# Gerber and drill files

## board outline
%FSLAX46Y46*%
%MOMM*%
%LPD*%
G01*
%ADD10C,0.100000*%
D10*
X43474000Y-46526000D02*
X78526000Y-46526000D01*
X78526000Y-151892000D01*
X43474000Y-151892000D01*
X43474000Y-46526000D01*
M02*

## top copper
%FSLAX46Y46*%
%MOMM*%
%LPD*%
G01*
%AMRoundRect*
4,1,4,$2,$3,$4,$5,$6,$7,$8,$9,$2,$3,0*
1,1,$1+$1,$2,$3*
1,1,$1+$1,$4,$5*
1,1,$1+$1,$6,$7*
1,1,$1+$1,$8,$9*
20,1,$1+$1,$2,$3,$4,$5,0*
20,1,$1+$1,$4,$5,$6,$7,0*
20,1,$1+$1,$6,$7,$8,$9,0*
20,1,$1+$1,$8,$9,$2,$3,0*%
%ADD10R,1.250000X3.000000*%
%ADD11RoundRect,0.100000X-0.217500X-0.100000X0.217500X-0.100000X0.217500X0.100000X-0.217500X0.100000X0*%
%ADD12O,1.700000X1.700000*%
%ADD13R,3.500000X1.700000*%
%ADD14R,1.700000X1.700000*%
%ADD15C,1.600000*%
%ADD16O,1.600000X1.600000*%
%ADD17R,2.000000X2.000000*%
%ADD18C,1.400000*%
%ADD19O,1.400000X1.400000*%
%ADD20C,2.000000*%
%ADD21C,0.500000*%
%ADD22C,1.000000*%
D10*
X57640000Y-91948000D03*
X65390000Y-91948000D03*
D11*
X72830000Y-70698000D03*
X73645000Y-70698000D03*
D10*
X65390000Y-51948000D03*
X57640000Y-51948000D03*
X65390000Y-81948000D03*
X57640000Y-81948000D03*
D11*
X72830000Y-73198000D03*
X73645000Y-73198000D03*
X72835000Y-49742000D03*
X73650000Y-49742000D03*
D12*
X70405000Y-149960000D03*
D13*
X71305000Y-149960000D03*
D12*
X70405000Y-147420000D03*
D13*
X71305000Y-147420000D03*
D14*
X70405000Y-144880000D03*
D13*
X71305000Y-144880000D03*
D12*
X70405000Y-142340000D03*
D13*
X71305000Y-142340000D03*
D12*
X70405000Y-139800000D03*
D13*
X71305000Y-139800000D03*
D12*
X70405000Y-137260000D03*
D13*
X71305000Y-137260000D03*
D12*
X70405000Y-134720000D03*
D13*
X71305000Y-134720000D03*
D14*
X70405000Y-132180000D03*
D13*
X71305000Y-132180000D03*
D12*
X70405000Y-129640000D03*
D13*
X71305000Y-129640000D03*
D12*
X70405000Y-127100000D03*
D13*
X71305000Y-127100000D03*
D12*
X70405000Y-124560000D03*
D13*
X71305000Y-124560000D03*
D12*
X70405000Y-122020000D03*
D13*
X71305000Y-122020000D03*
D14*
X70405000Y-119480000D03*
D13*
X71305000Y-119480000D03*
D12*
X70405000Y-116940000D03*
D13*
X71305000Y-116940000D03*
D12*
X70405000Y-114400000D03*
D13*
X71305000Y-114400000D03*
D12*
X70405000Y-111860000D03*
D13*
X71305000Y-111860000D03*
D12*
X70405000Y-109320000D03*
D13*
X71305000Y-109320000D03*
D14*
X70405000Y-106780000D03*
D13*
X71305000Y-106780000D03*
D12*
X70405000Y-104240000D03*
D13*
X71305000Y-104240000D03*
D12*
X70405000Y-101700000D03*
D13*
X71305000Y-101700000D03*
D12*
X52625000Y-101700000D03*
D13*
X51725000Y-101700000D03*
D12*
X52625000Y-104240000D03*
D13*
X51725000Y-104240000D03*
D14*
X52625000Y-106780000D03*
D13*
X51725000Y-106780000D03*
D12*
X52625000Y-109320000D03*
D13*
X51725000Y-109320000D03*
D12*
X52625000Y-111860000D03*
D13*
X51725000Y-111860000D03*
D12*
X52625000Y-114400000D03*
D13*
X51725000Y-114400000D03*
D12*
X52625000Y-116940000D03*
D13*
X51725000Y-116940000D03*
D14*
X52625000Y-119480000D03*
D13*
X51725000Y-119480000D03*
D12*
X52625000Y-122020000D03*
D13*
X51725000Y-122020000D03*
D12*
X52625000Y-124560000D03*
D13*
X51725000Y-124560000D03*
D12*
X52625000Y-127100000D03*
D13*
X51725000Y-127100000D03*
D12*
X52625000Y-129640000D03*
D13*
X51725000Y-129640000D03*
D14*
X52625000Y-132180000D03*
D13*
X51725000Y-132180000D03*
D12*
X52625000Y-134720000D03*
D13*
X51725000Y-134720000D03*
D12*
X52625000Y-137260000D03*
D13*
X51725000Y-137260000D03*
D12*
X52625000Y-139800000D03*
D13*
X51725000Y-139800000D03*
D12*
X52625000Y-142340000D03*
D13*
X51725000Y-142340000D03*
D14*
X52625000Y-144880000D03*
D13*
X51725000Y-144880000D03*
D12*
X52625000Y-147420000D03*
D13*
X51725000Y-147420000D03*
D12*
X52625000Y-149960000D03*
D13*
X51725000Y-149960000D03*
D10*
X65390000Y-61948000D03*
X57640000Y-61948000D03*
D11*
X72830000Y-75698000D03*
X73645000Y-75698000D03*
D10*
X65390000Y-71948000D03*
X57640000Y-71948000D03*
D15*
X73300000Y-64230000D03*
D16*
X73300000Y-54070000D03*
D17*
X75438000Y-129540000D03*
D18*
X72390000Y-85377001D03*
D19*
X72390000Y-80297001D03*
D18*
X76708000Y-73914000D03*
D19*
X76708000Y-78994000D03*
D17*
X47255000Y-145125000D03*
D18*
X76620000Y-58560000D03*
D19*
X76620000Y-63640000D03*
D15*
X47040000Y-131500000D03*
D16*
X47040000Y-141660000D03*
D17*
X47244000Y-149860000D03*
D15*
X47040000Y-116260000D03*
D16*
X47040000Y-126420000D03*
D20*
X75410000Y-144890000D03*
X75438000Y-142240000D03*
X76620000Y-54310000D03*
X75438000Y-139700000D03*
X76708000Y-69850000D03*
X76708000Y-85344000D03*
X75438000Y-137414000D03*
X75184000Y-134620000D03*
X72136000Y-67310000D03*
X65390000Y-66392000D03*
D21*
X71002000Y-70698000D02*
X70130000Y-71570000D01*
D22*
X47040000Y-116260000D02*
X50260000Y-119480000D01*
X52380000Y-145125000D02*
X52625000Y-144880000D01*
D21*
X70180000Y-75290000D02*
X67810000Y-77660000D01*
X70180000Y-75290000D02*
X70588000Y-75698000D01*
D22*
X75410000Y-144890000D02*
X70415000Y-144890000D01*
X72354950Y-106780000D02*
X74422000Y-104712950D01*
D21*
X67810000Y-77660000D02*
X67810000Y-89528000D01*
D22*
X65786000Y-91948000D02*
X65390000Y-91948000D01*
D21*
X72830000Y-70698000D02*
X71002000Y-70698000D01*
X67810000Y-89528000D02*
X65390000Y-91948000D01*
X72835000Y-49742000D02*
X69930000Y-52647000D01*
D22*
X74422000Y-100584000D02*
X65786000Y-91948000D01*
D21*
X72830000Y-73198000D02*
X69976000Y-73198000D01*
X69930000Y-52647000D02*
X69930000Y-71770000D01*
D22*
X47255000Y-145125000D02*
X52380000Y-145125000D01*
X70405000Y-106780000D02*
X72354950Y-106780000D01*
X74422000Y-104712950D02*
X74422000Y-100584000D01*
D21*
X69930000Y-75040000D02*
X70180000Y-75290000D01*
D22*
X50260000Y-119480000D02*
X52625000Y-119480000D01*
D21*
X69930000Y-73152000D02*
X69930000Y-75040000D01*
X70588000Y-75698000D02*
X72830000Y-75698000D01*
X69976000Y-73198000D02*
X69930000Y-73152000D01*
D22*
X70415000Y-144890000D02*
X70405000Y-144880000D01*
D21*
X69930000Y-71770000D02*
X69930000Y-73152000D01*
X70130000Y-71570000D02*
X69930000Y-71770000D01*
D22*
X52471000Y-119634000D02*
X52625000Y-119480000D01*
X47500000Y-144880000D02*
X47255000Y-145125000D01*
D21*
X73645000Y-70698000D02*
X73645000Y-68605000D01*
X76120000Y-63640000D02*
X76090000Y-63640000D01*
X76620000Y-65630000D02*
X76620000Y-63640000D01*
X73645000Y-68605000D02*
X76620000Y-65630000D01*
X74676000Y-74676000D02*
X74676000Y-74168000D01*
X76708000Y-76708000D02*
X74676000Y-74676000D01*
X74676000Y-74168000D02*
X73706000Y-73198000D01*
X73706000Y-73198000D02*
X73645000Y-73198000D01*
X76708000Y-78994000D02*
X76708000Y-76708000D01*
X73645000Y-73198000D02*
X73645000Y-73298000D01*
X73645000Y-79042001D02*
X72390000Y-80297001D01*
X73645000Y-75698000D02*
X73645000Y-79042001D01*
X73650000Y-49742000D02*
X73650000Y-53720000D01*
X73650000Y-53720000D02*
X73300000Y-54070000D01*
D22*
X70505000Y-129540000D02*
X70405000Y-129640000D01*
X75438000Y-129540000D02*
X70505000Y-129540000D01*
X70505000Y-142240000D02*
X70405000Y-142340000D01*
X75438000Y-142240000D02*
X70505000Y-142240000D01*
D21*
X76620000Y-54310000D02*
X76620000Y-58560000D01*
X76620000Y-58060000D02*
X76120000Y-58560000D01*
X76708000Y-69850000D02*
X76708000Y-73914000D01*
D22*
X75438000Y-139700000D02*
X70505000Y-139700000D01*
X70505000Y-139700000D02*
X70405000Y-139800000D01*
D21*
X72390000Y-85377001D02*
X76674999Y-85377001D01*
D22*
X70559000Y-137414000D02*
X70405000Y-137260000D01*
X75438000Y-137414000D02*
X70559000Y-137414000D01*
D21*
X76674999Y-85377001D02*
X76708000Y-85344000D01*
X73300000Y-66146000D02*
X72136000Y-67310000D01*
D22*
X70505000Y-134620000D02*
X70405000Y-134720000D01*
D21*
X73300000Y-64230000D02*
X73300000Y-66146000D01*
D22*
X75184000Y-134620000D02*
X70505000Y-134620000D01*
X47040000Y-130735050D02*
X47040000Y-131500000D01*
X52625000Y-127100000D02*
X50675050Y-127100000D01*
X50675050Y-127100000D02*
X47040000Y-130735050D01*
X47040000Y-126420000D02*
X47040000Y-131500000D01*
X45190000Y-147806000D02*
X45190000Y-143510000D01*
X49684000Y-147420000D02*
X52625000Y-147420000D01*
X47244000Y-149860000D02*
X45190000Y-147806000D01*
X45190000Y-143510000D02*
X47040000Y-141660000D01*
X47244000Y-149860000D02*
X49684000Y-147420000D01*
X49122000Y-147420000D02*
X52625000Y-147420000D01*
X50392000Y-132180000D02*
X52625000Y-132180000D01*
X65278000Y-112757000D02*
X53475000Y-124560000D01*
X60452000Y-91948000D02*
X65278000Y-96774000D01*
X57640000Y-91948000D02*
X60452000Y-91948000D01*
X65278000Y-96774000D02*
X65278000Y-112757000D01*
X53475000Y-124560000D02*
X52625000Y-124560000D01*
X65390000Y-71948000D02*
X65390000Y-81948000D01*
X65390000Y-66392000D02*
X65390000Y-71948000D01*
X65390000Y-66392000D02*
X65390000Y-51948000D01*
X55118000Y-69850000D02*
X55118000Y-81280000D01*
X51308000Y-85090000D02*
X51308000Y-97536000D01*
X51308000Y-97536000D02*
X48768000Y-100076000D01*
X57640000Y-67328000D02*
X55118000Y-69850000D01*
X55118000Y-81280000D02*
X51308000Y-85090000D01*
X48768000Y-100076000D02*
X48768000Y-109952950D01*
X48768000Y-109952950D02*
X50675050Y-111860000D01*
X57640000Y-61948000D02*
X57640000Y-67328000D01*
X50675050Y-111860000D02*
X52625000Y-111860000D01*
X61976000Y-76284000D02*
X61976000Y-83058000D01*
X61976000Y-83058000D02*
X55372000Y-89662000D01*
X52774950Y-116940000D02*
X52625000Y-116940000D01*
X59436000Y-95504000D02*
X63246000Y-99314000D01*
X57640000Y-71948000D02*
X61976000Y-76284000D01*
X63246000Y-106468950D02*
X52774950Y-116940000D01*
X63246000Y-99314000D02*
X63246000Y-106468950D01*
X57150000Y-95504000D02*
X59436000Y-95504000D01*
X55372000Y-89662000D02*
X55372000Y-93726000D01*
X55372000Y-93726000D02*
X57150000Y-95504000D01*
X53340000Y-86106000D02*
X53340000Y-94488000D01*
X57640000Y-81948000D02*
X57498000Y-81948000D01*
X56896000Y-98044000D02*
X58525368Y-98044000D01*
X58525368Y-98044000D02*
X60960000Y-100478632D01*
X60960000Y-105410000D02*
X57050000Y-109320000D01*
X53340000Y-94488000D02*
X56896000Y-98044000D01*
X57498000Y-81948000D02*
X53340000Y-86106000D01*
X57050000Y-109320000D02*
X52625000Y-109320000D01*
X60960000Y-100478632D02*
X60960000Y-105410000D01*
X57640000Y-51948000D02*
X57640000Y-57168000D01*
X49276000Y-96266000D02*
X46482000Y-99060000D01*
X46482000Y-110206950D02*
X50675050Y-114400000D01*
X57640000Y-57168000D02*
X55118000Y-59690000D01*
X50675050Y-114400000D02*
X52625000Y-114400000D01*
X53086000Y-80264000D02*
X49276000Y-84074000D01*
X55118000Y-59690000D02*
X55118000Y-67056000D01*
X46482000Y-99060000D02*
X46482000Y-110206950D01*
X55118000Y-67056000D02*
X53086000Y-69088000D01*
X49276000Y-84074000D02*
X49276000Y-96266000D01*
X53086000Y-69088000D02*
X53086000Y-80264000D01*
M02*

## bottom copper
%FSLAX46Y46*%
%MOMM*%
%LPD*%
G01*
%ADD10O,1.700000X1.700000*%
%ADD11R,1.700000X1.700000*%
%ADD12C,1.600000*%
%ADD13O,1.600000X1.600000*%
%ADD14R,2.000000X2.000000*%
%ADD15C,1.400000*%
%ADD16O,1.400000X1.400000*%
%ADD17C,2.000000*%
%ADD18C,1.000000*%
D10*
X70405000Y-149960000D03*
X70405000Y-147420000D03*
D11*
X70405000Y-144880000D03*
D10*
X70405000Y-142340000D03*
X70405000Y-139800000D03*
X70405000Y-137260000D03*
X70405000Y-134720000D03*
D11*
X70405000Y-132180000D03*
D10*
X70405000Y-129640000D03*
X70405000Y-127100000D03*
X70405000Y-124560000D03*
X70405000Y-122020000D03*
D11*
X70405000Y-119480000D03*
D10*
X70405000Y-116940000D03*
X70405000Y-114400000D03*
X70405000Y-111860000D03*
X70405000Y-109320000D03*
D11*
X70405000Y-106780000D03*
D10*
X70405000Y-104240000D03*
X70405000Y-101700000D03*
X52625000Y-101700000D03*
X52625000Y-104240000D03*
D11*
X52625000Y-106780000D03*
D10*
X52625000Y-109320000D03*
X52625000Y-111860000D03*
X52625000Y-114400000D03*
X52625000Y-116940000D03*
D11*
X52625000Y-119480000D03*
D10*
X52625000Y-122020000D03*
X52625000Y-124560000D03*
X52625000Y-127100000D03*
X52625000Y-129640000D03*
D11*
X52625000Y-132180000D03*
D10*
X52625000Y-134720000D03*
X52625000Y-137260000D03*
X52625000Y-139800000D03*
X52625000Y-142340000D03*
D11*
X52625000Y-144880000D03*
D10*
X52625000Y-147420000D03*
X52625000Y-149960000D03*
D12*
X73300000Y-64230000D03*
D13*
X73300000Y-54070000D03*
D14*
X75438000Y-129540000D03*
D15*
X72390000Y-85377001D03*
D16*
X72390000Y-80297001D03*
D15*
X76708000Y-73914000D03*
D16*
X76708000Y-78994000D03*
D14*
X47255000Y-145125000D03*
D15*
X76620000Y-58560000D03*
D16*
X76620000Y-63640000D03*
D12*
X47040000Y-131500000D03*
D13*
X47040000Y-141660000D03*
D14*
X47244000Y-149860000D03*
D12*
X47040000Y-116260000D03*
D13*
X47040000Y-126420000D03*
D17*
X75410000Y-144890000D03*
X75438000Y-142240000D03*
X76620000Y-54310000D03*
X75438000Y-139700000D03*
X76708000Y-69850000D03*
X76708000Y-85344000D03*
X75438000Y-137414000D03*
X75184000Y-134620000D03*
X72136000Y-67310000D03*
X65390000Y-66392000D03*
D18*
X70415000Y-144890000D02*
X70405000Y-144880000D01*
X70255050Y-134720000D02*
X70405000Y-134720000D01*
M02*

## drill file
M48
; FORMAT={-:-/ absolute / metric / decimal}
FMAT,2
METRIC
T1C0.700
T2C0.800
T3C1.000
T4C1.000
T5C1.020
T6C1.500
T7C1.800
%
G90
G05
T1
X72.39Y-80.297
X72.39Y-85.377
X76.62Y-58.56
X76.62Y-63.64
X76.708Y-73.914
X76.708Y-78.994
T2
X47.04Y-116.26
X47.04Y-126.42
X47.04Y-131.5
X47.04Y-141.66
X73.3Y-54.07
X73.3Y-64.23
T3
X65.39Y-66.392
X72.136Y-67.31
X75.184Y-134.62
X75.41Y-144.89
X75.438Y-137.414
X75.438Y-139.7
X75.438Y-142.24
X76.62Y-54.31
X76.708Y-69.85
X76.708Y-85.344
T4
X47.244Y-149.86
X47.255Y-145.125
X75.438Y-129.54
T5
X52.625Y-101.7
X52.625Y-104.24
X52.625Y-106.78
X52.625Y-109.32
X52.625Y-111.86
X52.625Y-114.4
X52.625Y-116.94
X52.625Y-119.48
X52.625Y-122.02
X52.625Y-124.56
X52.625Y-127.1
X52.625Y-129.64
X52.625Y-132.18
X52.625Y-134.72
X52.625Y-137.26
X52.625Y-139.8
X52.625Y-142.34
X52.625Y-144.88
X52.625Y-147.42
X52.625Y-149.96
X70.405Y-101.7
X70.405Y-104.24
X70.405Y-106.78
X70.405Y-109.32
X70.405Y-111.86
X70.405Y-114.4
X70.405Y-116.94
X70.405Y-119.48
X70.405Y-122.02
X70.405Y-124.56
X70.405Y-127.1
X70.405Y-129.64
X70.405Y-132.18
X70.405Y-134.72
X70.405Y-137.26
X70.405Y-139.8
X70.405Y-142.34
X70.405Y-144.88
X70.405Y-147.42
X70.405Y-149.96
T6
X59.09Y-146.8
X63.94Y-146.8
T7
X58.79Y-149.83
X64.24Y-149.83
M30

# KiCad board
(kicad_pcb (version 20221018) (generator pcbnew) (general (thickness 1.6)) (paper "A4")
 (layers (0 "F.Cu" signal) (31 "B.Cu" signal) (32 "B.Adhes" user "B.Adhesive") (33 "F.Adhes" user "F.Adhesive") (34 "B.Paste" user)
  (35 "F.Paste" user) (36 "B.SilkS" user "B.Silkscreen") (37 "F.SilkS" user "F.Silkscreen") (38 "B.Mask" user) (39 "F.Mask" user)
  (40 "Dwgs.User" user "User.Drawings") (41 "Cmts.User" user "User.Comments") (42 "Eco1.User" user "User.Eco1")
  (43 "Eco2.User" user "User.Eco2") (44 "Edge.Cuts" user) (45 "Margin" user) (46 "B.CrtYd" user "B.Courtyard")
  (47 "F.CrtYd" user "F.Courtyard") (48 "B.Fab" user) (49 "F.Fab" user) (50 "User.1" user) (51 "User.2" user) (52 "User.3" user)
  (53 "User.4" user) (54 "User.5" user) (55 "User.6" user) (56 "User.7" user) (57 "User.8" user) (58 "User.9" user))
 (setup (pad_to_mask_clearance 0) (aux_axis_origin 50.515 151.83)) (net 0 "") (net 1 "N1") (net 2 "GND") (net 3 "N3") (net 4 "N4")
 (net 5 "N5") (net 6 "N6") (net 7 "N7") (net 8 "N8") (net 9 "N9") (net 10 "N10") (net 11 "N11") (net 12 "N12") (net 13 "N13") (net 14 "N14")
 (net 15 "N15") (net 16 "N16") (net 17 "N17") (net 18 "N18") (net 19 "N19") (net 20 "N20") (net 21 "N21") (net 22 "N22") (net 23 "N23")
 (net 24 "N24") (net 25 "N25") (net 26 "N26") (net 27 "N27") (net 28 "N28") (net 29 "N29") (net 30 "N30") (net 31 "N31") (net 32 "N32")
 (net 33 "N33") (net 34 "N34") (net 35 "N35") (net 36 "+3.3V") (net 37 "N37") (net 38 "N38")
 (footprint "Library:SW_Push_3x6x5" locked (layer "F.Cu") (at 61.515 91.948)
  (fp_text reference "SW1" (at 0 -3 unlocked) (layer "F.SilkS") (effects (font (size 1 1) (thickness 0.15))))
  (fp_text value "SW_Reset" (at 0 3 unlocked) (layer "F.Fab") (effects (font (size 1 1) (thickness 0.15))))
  (pad "1" smd rect locked (at -3.875 0) (size 1.25 3) (layers "F.Cu" "F.Paste" "F.Mask") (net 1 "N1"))
  (pad "2" smd rect locked (at 3.875 0) (size 1.25 3) (layers "F.Cu" "F.Paste" "F.Mask") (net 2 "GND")))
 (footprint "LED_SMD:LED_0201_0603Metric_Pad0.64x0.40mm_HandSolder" (layer "F.Cu") (at 73.2375 70.698)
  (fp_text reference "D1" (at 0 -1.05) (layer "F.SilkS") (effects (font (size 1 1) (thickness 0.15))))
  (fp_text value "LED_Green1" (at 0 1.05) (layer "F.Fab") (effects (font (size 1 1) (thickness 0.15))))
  (pad "" smd roundrect (at -0.4325 0) (size 0.458 0.36) (layers "F.Paste") (roundrect_rratio 0.25))
  (pad "" smd roundrect (at 0.4325 0) (size 0.458 0.36) (layers "F.Paste") (roundrect_rratio 0.25))
  (pad "1" smd roundrect (at -0.4075 0) (size 0.635 0.4) (layers "F.Cu" "F.Mask") (roundrect_rratio 0.25) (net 2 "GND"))
  (pad "2" smd roundrect (at 0.4075 0) (size 0.635 0.4) (layers "F.Cu" "F.Mask") (roundrect_rratio 0.25) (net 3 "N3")))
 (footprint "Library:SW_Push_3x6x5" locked (layer "F.Cu") (at 61.515 51.948 180)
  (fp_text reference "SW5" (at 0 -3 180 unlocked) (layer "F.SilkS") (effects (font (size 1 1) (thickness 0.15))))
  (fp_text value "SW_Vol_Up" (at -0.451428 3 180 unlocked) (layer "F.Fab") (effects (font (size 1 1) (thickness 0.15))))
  (pad "1" smd rect locked (at -3.875 0 180) (size 1.25 3) (layers "F.Cu" "F.Paste" "F.Mask") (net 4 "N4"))
  (pad "2" smd rect locked (at 3.875 0 180) (size 1.25 3) (layers "F.Cu" "F.Paste" "F.Mask") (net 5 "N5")))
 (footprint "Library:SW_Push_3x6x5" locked (layer "F.Cu") (at 61.515 81.948 180)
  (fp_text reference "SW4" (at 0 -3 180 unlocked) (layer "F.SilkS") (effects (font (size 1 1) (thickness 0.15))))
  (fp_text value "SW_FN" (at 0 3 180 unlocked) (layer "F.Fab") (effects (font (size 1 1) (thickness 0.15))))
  (pad "1" smd rect locked (at -3.875 0 180) (size 1.25 3) (layers "F.Cu" "F.Paste" "F.Mask") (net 4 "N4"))
  (pad "2" smd rect locked (at 3.875 0 180) (size 1.25 3) (layers "F.Cu" "F.Paste" "F.Mask") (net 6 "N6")))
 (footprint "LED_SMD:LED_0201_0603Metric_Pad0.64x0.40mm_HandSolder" (layer "F.Cu") (at 73.2375 73.198)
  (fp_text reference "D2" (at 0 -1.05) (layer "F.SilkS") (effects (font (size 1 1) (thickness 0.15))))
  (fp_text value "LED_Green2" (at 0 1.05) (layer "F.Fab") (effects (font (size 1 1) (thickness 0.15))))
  (pad "" smd roundrect (at -0.4325 0) (size 0.458 0.36) (layers "F.Paste") (roundrect_rratio 0.25))
  (pad "" smd roundrect (at 0.4325 0) (size 0.458 0.36) (layers "F.Paste") (roundrect_rratio 0.25))
  (pad "1" smd roundrect (at -0.4075 0) (size 0.635 0.4) (layers "F.Cu" "F.Mask") (roundrect_rratio 0.25) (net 2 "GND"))
  (pad "2" smd roundrect (at 0.4075 0) (size 0.635 0.4) (layers "F.Cu" "F.Mask") (roundrect_rratio 0.25) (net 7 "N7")))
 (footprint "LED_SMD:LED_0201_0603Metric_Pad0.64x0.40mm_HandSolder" (layer "F.Cu") (at 73.2425 49.742)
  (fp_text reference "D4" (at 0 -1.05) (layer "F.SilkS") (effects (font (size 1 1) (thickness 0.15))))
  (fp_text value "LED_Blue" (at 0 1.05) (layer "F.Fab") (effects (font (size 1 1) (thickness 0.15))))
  (pad "" smd roundrect (at -0.4325 0) (size 0.458 0.36) (layers "F.Paste") (roundrect_rratio 0.25))
  (pad "" smd roundrect (at 0.4325 0) (size 0.458 0.36) (layers "F.Paste") (roundrect_rratio 0.25))
  (pad "1" smd roundrect (at -0.4075 0) (size 0.635 0.4) (layers "F.Cu" "F.Mask") (roundrect_rratio 0.25) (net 2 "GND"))
  (pad "2" smd roundrect (at 0.4075 0) (size 0.635 0.4) (layers "F.Cu" "F.Mask") (roundrect_rratio 0.25) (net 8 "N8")))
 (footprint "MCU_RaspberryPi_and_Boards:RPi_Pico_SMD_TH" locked (layer "F.Cu") (at 61.515 125.83 180)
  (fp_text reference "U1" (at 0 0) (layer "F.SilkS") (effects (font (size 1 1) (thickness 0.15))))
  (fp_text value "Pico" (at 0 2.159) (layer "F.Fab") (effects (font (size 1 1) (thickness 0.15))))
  (pad "" np_thru_hole oval locked (at -2.725 -24 180) (size 1.8 1.8) (drill 1.8) (layers "*.Cu" "*.Mask"))
  (pad "" np_thru_hole oval locked (at -2.425 -20.97 180) (size 1.5 1.5) (drill 1.5) (layers "*.Cu" "*.Mask"))
  (pad "" np_thru_hole oval locked (at 2.425 -20.97 180) (size 1.5 1.5) (drill 1.5) (layers "*.Cu" "*.Mask"))
  (pad "" np_thru_hole oval locked (at 2.725 -24 180) (size 1.8 1.8) (drill 1.8) (layers "*.Cu" "*.Mask"))
  (pad "1" thru_hole oval locked (at -8.89 -24.13 180) (size 1.7 1.7) (drill 1.02) (layers "*.Cu" "*.Mask") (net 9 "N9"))
  (pad "1" smd rect locked (at -8.89 -24.13 180) (size 3.5 1.7) (drill (offset -0.9 0)) (layers "F.Cu" "F.Mask") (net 9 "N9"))
  (pad "2" thru_hole oval locked (at -8.89 -21.59 180) (size 1.7 1.7) (drill 1.02) (layers "*.Cu" "*.Mask") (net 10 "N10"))
  (pad "2" smd rect locked (at -8.89 -21.59 180) (size 3.5 1.7) (drill (offset -0.9 0)) (layers "F.Cu" "F.Mask") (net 10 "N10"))
  (pad "3" thru_hole rect locked (at -8.89 -19.05 180) (size 1.7 1.7) (drill 1.02) (layers "*.Cu" "*.Mask") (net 2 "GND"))
  (pad "3" smd rect locked (at -8.89 -19.05 180) (size 3.5 1.7) (drill (offset -0.9 0)) (layers "F.Cu" "F.Mask") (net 2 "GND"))
  (pad "4" thru_hole oval locked (at -8.89 -16.51 180) (size 1.7 1.7) (drill 1.02) (layers "*.Cu" "*.Mask") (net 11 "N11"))
  (pad "4" smd rect locked (at -8.89 -16.51 180) (size 3.5 1.7) (drill (offset -0.9 0)) (layers "F.Cu" "F.Mask") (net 11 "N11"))
  (pad "5" thru_hole oval locked (at -8.89 -13.97 180) (size 1.7 1.7) (drill 1.02) (layers "*.Cu" "*.Mask") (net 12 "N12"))
  (pad "5" smd rect locked (at -8.89 -13.97 180) (size 3.5 1.7) (drill (offset -0.9 0)) (layers "F.Cu" "F.Mask") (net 12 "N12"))
  (pad "6" thru_hole oval locked (at -8.89 -11.43 180) (size 1.7 1.7) (drill 1.02) (layers "*.Cu" "*.Mask") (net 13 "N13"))
  (pad "6" smd rect locked (at -8.89 -11.43 180) (size 3.5 1.7) (drill (offset -0.9 0)) (layers "F.Cu" "F.Mask") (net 13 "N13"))
  (pad "7" thru_hole oval locked (at -8.89 -8.89 180) (size 1.7 1.7) (drill 1.02) (layers "*.Cu" "*.Mask") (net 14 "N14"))
  (pad "7" smd rect locked (at -8.89 -8.89 180) (size 3.5 1.7) (drill (offset -0.9 0)) (layers "F.Cu" "F.Mask") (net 14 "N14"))
  (pad "8" thru_hole rect locked (at -8.89 -6.35 180) (size 1.7 1.7) (drill 1.02) (layers "*.Cu" "*.Mask") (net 2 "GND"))
  (pad "8" smd rect locked (at -8.89 -6.35 180) (size 3.5 1.7) (drill (offset -0.9 0)) (layers "F.Cu" "F.Mask") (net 2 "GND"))
  (pad "9" thru_hole oval locked (at -8.89 -3.81 180) (size 1.7 1.7) (drill 1.02) (layers "*.Cu" "*.Mask") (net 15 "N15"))
  (pad "9" smd rect locked (at -8.89 -3.81 180) (size 3.5 1.7) (drill (offset -0.9 0)) (layers "F.Cu" "F.Mask") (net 15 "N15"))
  (pad "10" thru_hole oval locked (at -8.89 -1.27 180) (size 1.7 1.7) (drill 1.02) (layers "*.Cu" "*.Mask") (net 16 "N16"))
  (pad "10" smd rect locked (at -8.89 -1.27 180) (size 3.5 1.7) (drill (offset -0.9 0)) (layers "F.Cu" "F.Mask") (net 16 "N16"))
  (pad "11" thru_hole oval locked (at -8.89 1.27 180) (size 1.7 1.7) (drill 1.02) (layers "*.Cu" "*.Mask") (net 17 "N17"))
  (pad "11" smd rect locked (at -8.89 1.27 180) (size 3.5 1.7) (drill (offset -0.9 0)) (layers "F.Cu" "F.Mask") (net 17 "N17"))
  (pad "12" thru_hole oval locked (at -8.89 3.81 180) (size 1.7 1.7) (drill 1.02) (layers "*.Cu" "*.Mask") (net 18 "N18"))
  (pad "12" smd rect locked (at -8.89 3.81 180) (size 3.5 1.7) (drill (offset -0.9 0)) (layers "F.Cu" "F.Mask") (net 18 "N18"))
  (pad "13" thru_hole rect locked (at -8.89 6.35 180) (size 1.7 1.7) (drill 1.02) (layers "*.Cu" "*.Mask") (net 2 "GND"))
  (pad "13" smd rect locked (at -8.89 6.35 180) (size 3.5 1.7) (drill (offset -0.9 0)) (layers "F.Cu" "F.Mask") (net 2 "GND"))
  (pad "14" thru_hole oval locked (at -8.89 8.89 180) (size 1.7 1.7) (drill 1.02) (layers "*.Cu" "*.Mask") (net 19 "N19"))
  (pad "14" smd rect locked (at -8.89 8.89 180) (size 3.5 1.7) (drill (offset -0.9 0)) (layers "F.Cu" "F.Mask") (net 19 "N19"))
  (pad "15" thru_hole oval locked (at -8.89 11.43 180) (size 1.7 1.7) (drill 1.02) (layers "*.Cu" "*.Mask") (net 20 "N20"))
  (pad "15" smd rect locked (at -8.89 11.43 180) (size 3.5 1.7) (drill (offset -0.9 0)) (layers "F.Cu" "F.Mask") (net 20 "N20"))
  (pad "16" thru_hole oval locked (at -8.89 13.97 180) (size 1.7 1.7) (drill 1.02) (layers "*.Cu" "*.Mask") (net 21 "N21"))
  (pad "16" smd rect locked (at -8.89 13.97 180) (size 3.5 1.7) (drill (offset -0.9 0)) (layers "F.Cu" "F.Mask") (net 21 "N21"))
  (pad "17" thru_hole oval locked (at -8.89 16.51 180) (size 1.7 1.7) (drill 1.02) (layers "*.Cu" "*.Mask") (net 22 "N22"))
  (pad "17" smd rect locked (at -8.89 16.51 180) (size 3.5 1.7) (drill (offset -0.9 0)) (layers "F.Cu" "F.Mask") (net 22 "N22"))
  (pad "18" thru_hole rect locked (at -8.89 19.05 180) (size 1.7 1.7) (drill 1.02) (layers "*.Cu" "*.Mask") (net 2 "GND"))
  (pad "18" smd rect locked (at -8.89 19.05 180) (size 3.5 1.7) (drill (offset -0.9 0)) (layers "F.Cu" "F.Mask") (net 2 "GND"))
  (pad "19" thru_hole oval locked (at -8.89 21.59 180) (size 1.7 1.7) (drill 1.02) (layers "*.Cu" "*.Mask") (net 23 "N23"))
  (pad "19" smd rect locked (at -8.89 21.59 180) (size 3.5 1.7) (drill (offset -0.9 0)) (layers "F.Cu" "F.Mask") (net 23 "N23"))
  (pad "20" thru_hole oval locked (at -8.89 24.13 180) (size 1.7 1.7) (drill 1.02) (layers "*.Cu" "*.Mask") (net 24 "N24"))
  (pad "20" smd rect locked (at -8.89 24.13 180) (size 3.5 1.7) (drill (offset -0.9 0)) (layers "F.Cu" "F.Mask") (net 24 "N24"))
  (pad "21" thru_hole oval locked (at 8.89 24.13 180) (size 1.7 1.7) (drill 1.02) (layers "*.Cu" "*.Mask") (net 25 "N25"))
  (pad "21" smd rect locked (at 8.89 24.13 180) (size 3.5 1.7) (drill (offset 0.9 0)) (layers "F.Cu" "F.Mask") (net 25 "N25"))
  (pad "22" thru_hole oval locked (at 8.89 21.59 180) (size 1.7 1.7) (drill 1.02) (layers "*.Cu" "*.Mask") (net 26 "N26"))
  (pad "22" smd rect locked (at 8.89 21.59 180) (size 3.5 1.7) (drill (offset 0.9 0)) (layers "F.Cu" "F.Mask") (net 26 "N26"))
  (pad "23" thru_hole rect locked (at 8.89 19.05 180) (size 1.7 1.7) (drill 1.02) (layers "*.Cu" "*.Mask") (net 2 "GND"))
  (pad "23" smd rect locked (at 8.89 19.05 180) (size 3.5 1.7) (drill (offset 0.9 0)) (layers "F.Cu" "F.Mask") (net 2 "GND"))
  (pad "24" thru_hole oval locked (at 8.89 16.51 180) (size 1.7 1.7) (drill 1.02) (layers "*.Cu" "*.Mask") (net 6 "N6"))
  (pad "24" smd rect locked (at 8.89 16.51 180) (size 3.5 1.7) (drill (offset 0.9 0)) (layers "F.Cu" "F.Mask") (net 6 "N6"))
  (pad "25" thru_hole oval locked (at 8.89 13.97 180) (size 1.7 1.7) (drill 1.02) (layers "*.Cu" "*.Mask") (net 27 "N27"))
  (pad "25" smd rect locked (at 8.89 13.97 180) (size 3.5 1.7) (drill (offset 0.9 0)) (layers "F.Cu" "F.Mask") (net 27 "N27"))
  (pad "26" thru_hole oval locked (at 8.89 11.43 180) (size 1.7 1.7) (drill 1.02) (layers "*.Cu" "*.Mask") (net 5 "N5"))
  (pad "26" smd rect locked (at 8.89 11.43 180) (size 3.5 1.7) (drill (offset 0.9 0)) (layers "F.Cu" "F.Mask") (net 5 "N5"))
  (pad "27" thru_hole oval locked (at 8.89 8.89 180) (size 1.7 1.7) (drill 1.02) (layers "*.Cu" "*.Mask") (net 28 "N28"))
  (pad "27" smd rect locked (at 8.89 8.89 180) (size 3.5 1.7) (drill (offset 0.9 0)) (layers "F.Cu" "F.Mask") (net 28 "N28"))
  (pad "28" thru_hole rect locked (at 8.89 6.35 180) (size 1.7 1.7) (drill 1.02) (layers "*.Cu" "*.Mask") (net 2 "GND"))
  (pad "28" smd rect locked (at 8.89 6.35 180) (size 3.5 1.7) (drill (offset 0.9 0)) (layers "F.Cu" "F.Mask") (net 2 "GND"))
  (pad "29" thru_hole oval locked (at 8.89 3.81 180) (size 1.7 1.7) (drill 1.02) (layers "*.Cu" "*.Mask") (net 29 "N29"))
  (pad "29" smd rect locked (at 8.89 3.81 180) (size 3.5 1.7) (drill (offset 0.9 0)) (layers "F.Cu" "F.Mask") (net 29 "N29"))
  (pad "30" thru_hole oval locked (at 8.89 1.27 180) (size 1.7 1.7) (drill 1.02) (layers "*.Cu" "*.Mask") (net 1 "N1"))
  (pad "30" smd rect locked (at 8.89 1.27 180) (size 3.5 1.7) (drill (offset 0.9 0)) (layers "F.Cu" "F.Mask") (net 1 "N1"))
  (pad "31" thru_hole oval locked (at 8.89 -1.27 180) (size 1.7 1.7) (drill 1.02) (layers "*.Cu" "*.Mask") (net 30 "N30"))
  (pad "31" smd rect locked (at 8.89 -1.27 180) (size 3.5 1.7) (drill (offset 0.9 0)) (layers "F.Cu" "F.Mask") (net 30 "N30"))
  (pad "32" thru_hole oval locked (at 8.89 -3.81 180) (size 1.7 1.7) (drill 1.02) (layers "*.Cu" "*.Mask") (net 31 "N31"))
  (pad "32" smd rect locked (at 8.89 -3.81 180) (size 3.5 1.7) (drill (offset 0.9 0)) (layers "F.Cu" "F.Mask") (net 31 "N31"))
  (pad "33" thru_hole rect locked (at 8.89 -6.35 180) (size 1.7 1.7) (drill 1.02) (layers "*.Cu" "*.Mask") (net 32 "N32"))
  (pad "33" smd rect locked (at 8.89 -6.35 180) (size 3.5 1.7) (drill (offset 0.9 0)) (layers "F.Cu" "F.Mask") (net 32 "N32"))
  (pad "34" thru_hole oval locked (at 8.89 -8.89 180) (size 1.7 1.7) (drill 1.02) (layers "*.Cu" "*.Mask") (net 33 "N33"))
  (pad "34" smd rect locked (at 8.89 -8.89 180) (size 3.5 1.7) (drill (offset 0.9 0)) (layers "F.Cu" "F.Mask") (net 33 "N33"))
  (pad "35" thru_hole oval locked (at 8.89 -11.43 180) (size 1.7 1.7) (drill 1.02) (layers "*.Cu" "*.Mask") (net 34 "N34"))
  (pad "35" smd rect locked (at 8.89 -11.43 180) (size 3.5 1.7) (drill (offset 0.9 0)) (layers "F.Cu" "F.Mask") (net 34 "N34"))
  (pad "36" thru_hole oval locked (at 8.89 -13.97 180) (size 1.7 1.7) (drill 1.02) (layers "*.Cu" "*.Mask") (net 4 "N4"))
  (pad "36" smd rect locked (at 8.89 -13.97 180) (size 3.5 1.7) (drill (offset 0.9 0)) (layers "F.Cu" "F.Mask") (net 4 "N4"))
  (pad "37" thru_hole oval locked (at 8.89 -16.51 180) (size 1.7 1.7) (drill 1.02) (layers "*.Cu" "*.Mask") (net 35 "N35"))
  (pad "37" smd rect locked (at 8.89 -16.51 180) (size 3.5 1.7) (drill (offset 0.9 0)) (layers "F.Cu" "F.Mask") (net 35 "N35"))
  (pad "38" thru_hole rect locked (at 8.89 -19.05 180) (size 1.7 1.7) (drill 1.02) (layers "*.Cu" "*.Mask") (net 2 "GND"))
  (pad "38" smd rect locked (at 8.89 -19.05 180) (size 3.5 1.7) (drill (offset 0.9 0)) (layers "F.Cu" "F.Mask") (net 2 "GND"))
  (pad "39" thru_hole oval locked (at 8.89 -21.59 180) (size 1.7 1.7) (drill 1.02) (layers "*.Cu" "*.Mask") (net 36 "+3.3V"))
  (pad "39" smd rect locked (at 8.89 -21.59 180) (size 3.5 1.7) (drill (offset 0.9 0)) (layers "F.Cu" "F.Mask") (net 36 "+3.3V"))
  (pad "40" thru_hole oval locked (at 8.89 -24.13 180) (size 1.7 1.7) (drill 1.02) (layers "*.Cu" "*.Mask") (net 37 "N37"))
  (pad "40" smd rect locked (at 8.89 -24.13 180) (size 3.5 1.7) (drill (offset 0.9 0)) (layers "F.Cu" "F.Mask") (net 37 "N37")))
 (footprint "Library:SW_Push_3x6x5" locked (layer "F.Cu") (at 61.515 61.948 180)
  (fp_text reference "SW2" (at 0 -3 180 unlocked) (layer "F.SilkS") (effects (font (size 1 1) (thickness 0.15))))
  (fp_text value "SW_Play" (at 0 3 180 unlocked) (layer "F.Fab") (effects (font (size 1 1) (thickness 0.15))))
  (pad "1" smd rect locked (at -3.875 0 180) (size 1.25 3) (layers "F.Cu" "F.Paste" "F.Mask") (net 4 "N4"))
  (pad "2" smd rect locked (at 3.875 0 180) (size 1.25 3) (layers "F.Cu" "F.Paste" "F.Mask") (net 27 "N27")))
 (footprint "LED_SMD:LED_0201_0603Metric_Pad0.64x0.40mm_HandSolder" (layer "F.Cu") (at 73.2375 75.698)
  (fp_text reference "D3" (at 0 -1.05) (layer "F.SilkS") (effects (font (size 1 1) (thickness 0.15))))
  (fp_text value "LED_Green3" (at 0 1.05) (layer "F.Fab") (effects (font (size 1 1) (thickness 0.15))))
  (pad "" smd roundrect (at -0.4325 0) (size 0.458 0.36) (layers "F.Paste") (roundrect_rratio 0.25))
  (pad "" smd roundrect (at 0.4325 0) (size 0.458 0.36) (layers "F.Paste") (roundrect_rratio 0.25))
  (pad "1" smd roundrect (at -0.4075 0) (size 0.635 0.4) (layers "F.Cu" "F.Mask") (roundrect_rratio 0.25) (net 2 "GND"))
  (pad "2" smd roundrect (at 0.4075 0) (size 0.635 0.4) (layers "F.Cu" "F.Mask") (roundrect_rratio 0.25) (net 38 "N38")))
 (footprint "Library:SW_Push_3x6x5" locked (layer "F.Cu") (at 61.515 71.948 180)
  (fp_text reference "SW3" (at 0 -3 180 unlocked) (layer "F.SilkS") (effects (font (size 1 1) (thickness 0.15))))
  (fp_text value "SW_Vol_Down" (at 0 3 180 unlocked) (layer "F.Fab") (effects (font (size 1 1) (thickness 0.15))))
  (pad "1" smd rect locked (at -3.875 0 180) (size 1.25 3) (layers "F.Cu" "F.Paste" "F.Mask") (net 4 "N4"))
  (pad "2" smd rect locked (at 3.875 0 180) (size 1.25 3) (layers "F.Cu" "F.Paste" "F.Mask") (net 28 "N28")))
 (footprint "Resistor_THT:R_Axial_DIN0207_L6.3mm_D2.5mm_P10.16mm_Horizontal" (layer "B.Cu") (at 73.3 64.23 90)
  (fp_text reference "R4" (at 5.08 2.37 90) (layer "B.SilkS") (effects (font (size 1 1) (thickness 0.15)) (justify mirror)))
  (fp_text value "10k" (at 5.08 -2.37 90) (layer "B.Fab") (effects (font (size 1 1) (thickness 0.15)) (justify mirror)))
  (pad "1" thru_hole circle (at 0 0 90) (size 1.6 1.6) (drill 0.8) (layers "*.Cu" "*.Mask") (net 14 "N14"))
  (pad "2" thru_hole oval (at 10.16 0 90) (size 1.6 1.6) (drill 0.8) (layers "*.Cu" "*.Mask") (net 8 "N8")))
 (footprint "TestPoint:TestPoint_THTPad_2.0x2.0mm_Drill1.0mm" (layer "B.Cu") (at 75.438 129.54 180)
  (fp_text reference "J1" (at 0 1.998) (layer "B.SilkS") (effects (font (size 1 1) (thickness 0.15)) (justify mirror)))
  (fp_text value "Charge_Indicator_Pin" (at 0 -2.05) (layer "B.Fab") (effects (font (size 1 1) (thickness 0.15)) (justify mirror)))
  (pad "1" thru_hole rect (at 0 0 180) (size 2 2) (drill 1) (layers "*.Cu" "*.Mask") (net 15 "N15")))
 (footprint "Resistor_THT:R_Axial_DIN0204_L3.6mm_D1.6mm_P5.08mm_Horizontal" (layer "B.Cu") (at 72.39 85.377001 90)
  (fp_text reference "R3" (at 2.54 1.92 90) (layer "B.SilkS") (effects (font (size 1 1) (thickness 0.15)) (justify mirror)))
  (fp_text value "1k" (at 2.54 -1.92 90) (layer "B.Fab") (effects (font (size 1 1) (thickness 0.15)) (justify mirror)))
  (pad "1" thru_hole circle (at 0 0 90) (size 1.4 1.4) (drill 0.7) (layers "*.Cu" "*.Mask") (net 13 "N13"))
  (pad "2" thru_hole oval (at 5.08 0 90) (size 1.4 1.4) (drill 0.7) (layers "*.Cu" "*.Mask") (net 38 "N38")))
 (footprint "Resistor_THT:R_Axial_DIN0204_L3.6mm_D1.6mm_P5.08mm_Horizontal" (layer "B.Cu") (at 76.708 73.914 -90)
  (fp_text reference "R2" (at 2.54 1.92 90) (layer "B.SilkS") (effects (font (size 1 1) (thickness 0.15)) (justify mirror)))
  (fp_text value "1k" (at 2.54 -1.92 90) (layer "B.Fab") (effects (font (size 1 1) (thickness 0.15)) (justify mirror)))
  (pad "1" thru_hole circle (at 0 0 270) (size 1.4 1.4) (drill 0.7) (layers "*.Cu" "*.Mask") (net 12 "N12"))
  (pad "2" thru_hole oval (at 5.08 0 270) (size 1.4 1.4) (drill 0.7) (layers "*.Cu" "*.Mask") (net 7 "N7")))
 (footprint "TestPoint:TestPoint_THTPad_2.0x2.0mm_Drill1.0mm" (layer "B.Cu") (at 47.255 145.125 180)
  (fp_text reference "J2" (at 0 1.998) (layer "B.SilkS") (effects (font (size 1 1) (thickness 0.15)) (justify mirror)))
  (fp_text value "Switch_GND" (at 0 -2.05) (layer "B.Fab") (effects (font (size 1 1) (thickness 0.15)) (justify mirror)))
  (pad "1" thru_hole rect (at 0 0 180) (size 2 2) (drill 1) (layers "*.Cu" "*.Mask") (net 2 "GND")))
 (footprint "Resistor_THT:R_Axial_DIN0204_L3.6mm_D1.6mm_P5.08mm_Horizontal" (layer "B.Cu") (at 76.62 58.56 -90)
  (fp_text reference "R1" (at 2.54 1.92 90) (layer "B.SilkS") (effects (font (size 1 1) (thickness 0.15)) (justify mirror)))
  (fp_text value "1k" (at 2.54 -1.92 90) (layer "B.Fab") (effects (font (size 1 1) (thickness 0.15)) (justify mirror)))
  (pad "1" thru_hole circle (at 0 0 270) (size 1.4 1.4) (drill 0.7) (layers "*.Cu" "*.Mask") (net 11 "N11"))
  (pad "2" thru_hole oval (at 5.08 0 270) (size 1.4 1.4) (drill 0.7) (layers "*.Cu" "*.Mask") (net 3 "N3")))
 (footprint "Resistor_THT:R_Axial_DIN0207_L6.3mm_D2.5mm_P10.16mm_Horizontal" (layer "B.Cu") (at 47.04 131.5 -90)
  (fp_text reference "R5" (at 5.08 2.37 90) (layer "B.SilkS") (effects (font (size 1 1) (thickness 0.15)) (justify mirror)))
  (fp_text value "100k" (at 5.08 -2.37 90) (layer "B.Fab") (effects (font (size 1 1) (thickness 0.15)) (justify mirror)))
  (pad "1" thru_hole circle (at 0 0 270) (size 1.6 1.6) (drill 0.8) (layers "*.Cu" "*.Mask") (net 30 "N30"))
  (pad "2" thru_hole oval (at 10.16 0 270) (size 1.6 1.6) (drill 0.8) (layers "*.Cu" "*.Mask") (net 36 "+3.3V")))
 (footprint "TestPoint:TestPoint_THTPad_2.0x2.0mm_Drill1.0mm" (layer "B.Cu") (at 47.244 149.86 180)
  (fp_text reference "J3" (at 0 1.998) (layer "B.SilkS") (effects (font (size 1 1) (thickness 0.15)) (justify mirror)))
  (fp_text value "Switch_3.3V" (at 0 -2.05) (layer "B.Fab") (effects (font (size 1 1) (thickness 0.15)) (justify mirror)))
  (pad "1" thru_hole rect (at 0 0 180) (size 2 2) (drill 1) (layers "*.Cu" "*.Mask") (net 36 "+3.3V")))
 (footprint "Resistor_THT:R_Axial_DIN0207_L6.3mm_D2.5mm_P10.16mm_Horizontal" (layer "B.Cu") (at 47.04 116.26 -90)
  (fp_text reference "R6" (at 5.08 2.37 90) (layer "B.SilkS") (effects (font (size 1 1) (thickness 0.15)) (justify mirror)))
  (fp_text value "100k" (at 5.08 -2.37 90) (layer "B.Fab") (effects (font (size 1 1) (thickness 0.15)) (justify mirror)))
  (pad "1" thru_hole circle (at 0 0 270) (size 1.6 1.6) (drill 0.8) (layers "*.Cu" "*.Mask") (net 2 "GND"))
  (pad "2" thru_hole oval (at 10.16 0 270) (size 1.6 1.6) (drill 0.8) (layers "*.Cu" "*.Mask") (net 30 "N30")))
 (gr_rect (start 43.474 46.526) (end 78.526 151.892) (stroke (width 0.1) (type default)) (fill none) (layer "Edge.Cuts"))
 (segment (start 71.002 70.698) (end 70.13 71.57) (width 0.5) (layer "F.Cu") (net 2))
 (segment (start 47.04 116.26) (end 50.26 119.48) (width 1) (layer "F.Cu") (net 2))
 (segment (start 52.38 145.125) (end 52.625 144.88) (width 1) (layer "F.Cu") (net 2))
 (segment (start 70.18 75.29) (end 67.81 77.66) (width 0.5) (layer "F.Cu") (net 2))
 (segment (start 70.18 75.29) (end 70.588 75.698) (width 0.5) (layer "F.Cu") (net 2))
 (segment (start 75.41 144.89) (end 70.415 144.89) (width 1) (layer "F.Cu") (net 2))
 (segment (start 72.35495 106.78) (end 74.422 104.71295) (width 1) (layer "F.Cu") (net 2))
 (segment (start 67.81 77.66) (end 67.81 89.528) (width 0.5) (layer "F.Cu") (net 2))
 (segment (start 65.786 91.948) (end 65.39 91.948) (width 1) (layer "F.Cu") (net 2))
 (segment (start 72.83 70.698) (end 71.002 70.698) (width 0.5) (layer "F.Cu") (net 2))
 (segment (start 67.81 89.528) (end 65.39 91.948) (width 0.5) (layer "F.Cu") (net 2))
 (segment (start 72.835 49.742) (end 69.93 52.647) (width 0.5) (layer "F.Cu") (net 2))
 (segment (start 74.422 100.584) (end 65.786 91.948) (width 1) (layer "F.Cu") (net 2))
 (segment (start 72.83 73.198) (end 69.976 73.198) (width 0.5) (layer "F.Cu") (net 2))
 (segment (start 69.93 52.647) (end 69.93 71.77) (width 0.5) (layer "F.Cu") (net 2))
 (segment (start 47.255 145.125) (end 52.38 145.125) (width 1) (layer "F.Cu") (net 2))
 (segment (start 70.405 106.78) (end 72.35495 106.78) (width 1) (layer "F.Cu") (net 2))
 (segment (start 74.422 104.71295) (end 74.422 100.584) (width 1) (layer "F.Cu") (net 2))
 (segment (start 69.93 75.04) (end 70.18 75.29) (width 0.5) (layer "F.Cu") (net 2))
 (segment (start 50.26 119.48) (end 52.625 119.48) (width 1) (layer "F.Cu") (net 2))
 (segment (start 69.93 73.152) (end 69.93 75.04) (width 0.5) (layer "F.Cu") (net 2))
 (segment (start 70.588 75.698) (end 72.83 75.698) (width 0.5) (layer "F.Cu") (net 2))
 (segment (start 69.976 73.198) (end 69.93 73.152) (width 0.5) (layer "F.Cu") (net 2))
 (segment (start 70.415 144.89) (end 70.405 144.88) (width 1) (layer "F.Cu") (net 2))
 (segment (start 69.93 71.77) (end 69.93 73.152) (width 0.5) (layer "F.Cu") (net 2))
 (segment (start 70.13 71.57) (end 69.93 71.77) (width 0.5) (layer "F.Cu") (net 2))
 (segment (start 52.471 119.634) (end 52.625 119.48) (width 1) (layer "F.Cu") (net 2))
 (segment (start 47.5 144.88) (end 47.255 145.125) (width 1) (layer "F.Cu") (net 2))
 (via (at 75.41 144.89) (size 2) (drill 1) (layers "F.Cu" "B.Cu") (free) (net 2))
 (segment (start 70.415 144.89) (end 70.405 144.88) (width 1) (layer "B.Cu") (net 2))
 (segment (start 73.645 70.698) (end 73.645 68.605) (width 0.5) (layer "F.Cu") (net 3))
 (segment (start 76.12 63.64) (end 76.09 63.64) (width 0.5) (layer "F.Cu") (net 3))
 (segment (start 76.62 65.63) (end 76.62 63.64) (width 0.5) (layer "F.Cu") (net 3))
 (segment (start 73.645 68.605) (end 76.62 65.63) (width 0.5) (layer "F.Cu") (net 3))
 (segment (start 74.676 74.676) (end 74.676 74.168) (width 0.5) (layer "F.Cu") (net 7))
 (segment (start 76.708 76.708) (end 74.676 74.676) (width 0.5) (layer "F.Cu") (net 7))
 (segment (start 74.676 74.168) (end 73.706 73.198) (width 0.5) (layer "F.Cu") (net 7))
 (segment (start 73.706 73.198) (end 73.645 73.198) (width 0.5) (layer "F.Cu") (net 7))
 (segment (start 76.708 78.994) (end 76.708 76.708) (width 0.5) (layer "F.Cu") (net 7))
 (segment (start 73.645 73.198) (end 73.645 73.298) (width 0.5) (layer "F.Cu") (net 7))
 (segment (start 73.645 79.042001) (end 72.39 80.297001) (width 0.5) (layer "F.Cu") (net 38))
 (segment (start 73.645 75.698) (end 73.645 79.042001) (width 0.5) (layer "F.Cu") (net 38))
 (segment (start 73.65 49.742) (end 73.65 53.72) (width 0.5) (layer "F.Cu") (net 8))
 (segment (start 73.65 53.72) (end 73.3 54.07) (width 0.5) (layer "F.Cu") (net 8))
 (segment (start 70.505 129.54) (end 70.405 129.64) (width 1) (layer "F.Cu") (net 15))
 (segment (start 75.438 129.54) (end 70.505 129.54) (width 1) (layer "F.Cu") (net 15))
 (segment (start 70.505 142.24) (end 70.405 142.34) (width 1) (layer "F.Cu") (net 11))
 (segment (start 75.438 142.24) (end 70.505 142.24) (width 1) (layer "F.Cu") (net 11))
 (segment (start 76.62 54.31) (end 76.62 58.56) (width 0.5) (layer "F.Cu") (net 11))
 (segment (start 76.62 58.06) (end 76.12 58.56) (width 0.5) (layer "F.Cu") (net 11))
 (via (at 75.438 142.24) (size 2) (drill 1) (layers "F.Cu" "B.Cu") (free) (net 11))
 (via (at 76.62 54.31) (size 2) (drill 1) (layers "F.Cu" "B.Cu") (free) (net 11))
 (segment (start 76.708 69.85) (end 76.708 73.914) (width 0.5) (layer "F.Cu") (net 12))
 (segment (start 75.438 139.7) (end 70.505 139.7) (width 1) (layer "F.Cu") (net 12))
 (segment (start 70.505 139.7) (end 70.405 139.8) (width 1) (layer "F.Cu") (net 12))
 (via (at 75.438 139.7) (size 2) (drill 1) (layers "F.Cu" "B.Cu") (free) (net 12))
 (via (at 76.708 69.85) (size 2) (drill 1) (layers "F.Cu" "B.Cu") (free) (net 12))
 (segment (start 72.39 85.377001) (end 76.674999 85.377001) (width 0.5) (layer "F.Cu") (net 13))
 (segment (start 70.559 137.414) (end 70.405 137.26) (width 1) (layer "F.Cu") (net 13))
 (segment (start 75.438 137.414) (end 70.559 137.414) (width 1) (layer "F.Cu") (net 13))
 (segment (start 76.674999 85.377001) (end 76.708 85.344) (width 0.5) (layer "F.Cu") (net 13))
 (via (at 76.708 85.344) (size 2) (drill 1) (layers "F.Cu" "B.Cu") (free) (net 13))
 (via (at 75.438 137.414) (size 2) (drill 1) (layers "F.Cu" "B.Cu") (free) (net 13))
 (segment (start 73.3 66.146) (end 72.136 67.31) (width 0.5) (layer "F.Cu") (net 14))
 (segment (start 70.505 134.62) (end 70.405 134.72) (width 1) (layer "F.Cu") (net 14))
 (segment (start 73.3 64.23) (end 73.3 66.146) (width 0.5) (layer "F.Cu") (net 14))
 (segment (start 75.184 134.62) (end 70.505 134.62) (width 1) (layer "F.Cu") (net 14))
 (via (at 75.184 134.62) (size 2) (drill 1) (layers "F.Cu" "B.Cu") (free) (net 14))
 (via (at 72.136 67.31) (size 2) (drill 1) (layers "F.Cu" "B.Cu") (free) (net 14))
 (segment (start 70.25505 134.72) (end 70.405 134.72) (width 1) (layer "B.Cu") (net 14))
 (segment (start 47.04 130.73505) (end 47.04 131.5) (width 1) (layer "F.Cu") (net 30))
 (segment (start 52.625 127.1) (end 50.67505 127.1) (width 1) (layer "F.Cu") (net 30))
 (segment (start 50.67505 127.1) (end 47.04 130.73505) (width 1) (layer "F.Cu") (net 30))
 (segment (start 47.04 126.42) (end 47.04 131.5) (width 1) (layer "F.Cu") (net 30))
 (segment (start 45.19 147.806) (end 45.19 143.51) (width 1) (layer "F.Cu") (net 36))
 (segment (start 49.684 147.42) (end 52.625 147.42) (width 1) (layer "F.Cu") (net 36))
 (segment (start 47.244 149.86) (end 45.19 147.806) (width 1) (layer "F.Cu") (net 36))
 (segment (start 45.19 143.51) (end 47.04 141.66) (width 1) (layer "F.Cu") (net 36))
 (segment (start 47.244 149.86) (end 49.684 147.42) (width 1) (layer "F.Cu") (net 36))
 (segment (start 49.122 147.42) (end 52.625 147.42) (width 1) (layer "F.Cu") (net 36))
 (segment (start 50.392 132.18) (end 52.625 132.18) (width 1) (layer "F.Cu") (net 32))
 (segment (start 65.278 112.757) (end 53.475 124.56) (width 1) (layer "F.Cu") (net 1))
 (segment (start 60.452 91.948) (end 65.278 96.774) (width 1) (layer "F.Cu") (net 1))
 (segment (start 57.64 91.948) (end 60.452 91.948) (width 1) (layer "F.Cu") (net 1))
 (segment (start 65.278 96.774) (end 65.278 112.757) (width 1) (layer "F.Cu") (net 1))
 (segment (start 53.475 124.56) (end 52.625 124.56) (width 1) (layer "F.Cu") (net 1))
 (segment (start 65.39 71.948) (end 65.39 81.948) (width 1) (layer "F.Cu") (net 4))
 (segment (start 65.39 66.392) (end 65.39 71.948) (width 1) (layer "F.Cu") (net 4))
 (segment (start 65.39 66.392) (end 65.39 51.948) (width 1) (layer "F.Cu") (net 4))
 (via (at 65.39 66.392) (size 2) (drill 1) (layers "F.Cu" "B.Cu") (free) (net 4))
 (segment (start 55.118 69.85) (end 55.118 81.28) (width 1) (layer "F.Cu") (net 27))
 (segment (start 51.308 85.09) (end 51.308 97.536) (width 1) (layer "F.Cu") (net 27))
 (segment (start 51.308 97.536) (end 48.768 100.076) (width 1) (layer "F.Cu") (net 27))
 (segment (start 57.64 67.328) (end 55.118 69.85) (width 1) (layer "F.Cu") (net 27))
 (segment (start 55.118 81.28) (end 51.308 85.09) (width 1) (layer "F.Cu") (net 27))
 (segment (start 48.768 100.076) (end 48.768 109.95295) (width 1) (layer "F.Cu") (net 27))
 (segment (start 48.768 109.95295) (end 50.67505 111.86) (width 1) (layer "F.Cu") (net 27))
 (segment (start 57.64 61.948) (end 57.64 67.328) (width 1) (layer "F.Cu") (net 27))
 (segment (start 50.67505 111.86) (end 52.625 111.86) (width 1) (layer "F.Cu") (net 27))
 (segment (start 61.976 76.284) (end 61.976 83.058) (width 1) (layer "F.Cu") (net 28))
 (segment (start 61.976 83.058) (end 55.372 89.662) (width 1) (layer "F.Cu") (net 28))
 (segment (start 52.77495 116.94) (end 52.625 116.94) (width 1) (layer "F.Cu") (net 28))
 (segment (start 59.436 95.504) (end 63.246 99.314) (width 1) (layer "F.Cu") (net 28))
 (segment (start 57.64 71.948) (end 61.976 76.284) (width 1) (layer "F.Cu") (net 28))
 (segment (start 63.246 106.46895) (end 52.77495 116.94) (width 1) (layer "F.Cu") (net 28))
 (segment (start 63.246 99.314) (end 63.246 106.46895) (width 1) (layer "F.Cu") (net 28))
 (segment (start 57.15 95.504) (end 59.436 95.504) (width 1) (layer "F.Cu") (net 28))
 (segment (start 55.372 89.662) (end 55.372 93.726) (width 1) (layer "F.Cu") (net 28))
 (segment (start 55.372 93.726) (end 57.15 95.504) (width 1) (layer "F.Cu") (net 28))
 (segment (start 53.34 86.106) (end 53.34 94.488) (width 1) (layer "F.Cu") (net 6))
 (segment (start 57.64 81.948) (end 57.498 81.948) (width 1) (layer "F.Cu") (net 6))
 (segment (start 56.896 98.044) (end 58.525368 98.044) (width 1) (layer "F.Cu") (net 6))
 (segment (start 58.525368 98.044) (end 60.96 100.478632) (width 1) (layer "F.Cu") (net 6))
 (segment (start 60.96 105.41) (end 57.05 109.32) (width 1) (layer "F.Cu") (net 6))
 (segment (start 53.34 94.488) (end 56.896 98.044) (width 1) (layer "F.Cu") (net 6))
 (segment (start 57.498 81.948) (end 53.34 86.106) (width 1) (layer "F.Cu") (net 6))
 (segment (start 57.05 109.32) (end 52.625 109.32) (width 1) (layer "F.Cu") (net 6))
 (segment (start 60.96 100.478632) (end 60.96 105.41) (width 1) (layer "F.Cu") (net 6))
 (segment (start 57.64 51.948) (end 57.64 57.168) (width 1) (layer "F.Cu") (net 5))
 (segment (start 49.276 96.266) (end 46.482 99.06) (width 1) (layer "F.Cu") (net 5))
 (segment (start 46.482 110.20695) (end 50.67505 114.4) (width 1) (layer "F.Cu") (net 5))
 (segment (start 57.64 57.168) (end 55.118 59.69) (width 1) (layer "F.Cu") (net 5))
 (segment (start 50.67505 114.4) (end 52.625 114.4) (width 1) (layer "F.Cu") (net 5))
 (segment (start 53.086 80.264) (end 49.276 84.074) (width 1) (layer "F.Cu") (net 5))
 (segment (start 55.118 59.69) (end 55.118 67.056) (width 1) (layer "F.Cu") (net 5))
 (segment (start 46.482 99.06) (end 46.482 110.20695) (width 1) (layer "F.Cu") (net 5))
 (segment (start 55.118 67.056) (end 53.086 69.088) (width 1) (layer "F.Cu") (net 5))
 (segment (start 49.276 84.074) (end 49.276 96.266) (width 1) (layer "F.Cu") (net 5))
 (segment (start 53.086 69.088) (end 53.086 80.264) (width 1) (layer "F.Cu") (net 5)))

